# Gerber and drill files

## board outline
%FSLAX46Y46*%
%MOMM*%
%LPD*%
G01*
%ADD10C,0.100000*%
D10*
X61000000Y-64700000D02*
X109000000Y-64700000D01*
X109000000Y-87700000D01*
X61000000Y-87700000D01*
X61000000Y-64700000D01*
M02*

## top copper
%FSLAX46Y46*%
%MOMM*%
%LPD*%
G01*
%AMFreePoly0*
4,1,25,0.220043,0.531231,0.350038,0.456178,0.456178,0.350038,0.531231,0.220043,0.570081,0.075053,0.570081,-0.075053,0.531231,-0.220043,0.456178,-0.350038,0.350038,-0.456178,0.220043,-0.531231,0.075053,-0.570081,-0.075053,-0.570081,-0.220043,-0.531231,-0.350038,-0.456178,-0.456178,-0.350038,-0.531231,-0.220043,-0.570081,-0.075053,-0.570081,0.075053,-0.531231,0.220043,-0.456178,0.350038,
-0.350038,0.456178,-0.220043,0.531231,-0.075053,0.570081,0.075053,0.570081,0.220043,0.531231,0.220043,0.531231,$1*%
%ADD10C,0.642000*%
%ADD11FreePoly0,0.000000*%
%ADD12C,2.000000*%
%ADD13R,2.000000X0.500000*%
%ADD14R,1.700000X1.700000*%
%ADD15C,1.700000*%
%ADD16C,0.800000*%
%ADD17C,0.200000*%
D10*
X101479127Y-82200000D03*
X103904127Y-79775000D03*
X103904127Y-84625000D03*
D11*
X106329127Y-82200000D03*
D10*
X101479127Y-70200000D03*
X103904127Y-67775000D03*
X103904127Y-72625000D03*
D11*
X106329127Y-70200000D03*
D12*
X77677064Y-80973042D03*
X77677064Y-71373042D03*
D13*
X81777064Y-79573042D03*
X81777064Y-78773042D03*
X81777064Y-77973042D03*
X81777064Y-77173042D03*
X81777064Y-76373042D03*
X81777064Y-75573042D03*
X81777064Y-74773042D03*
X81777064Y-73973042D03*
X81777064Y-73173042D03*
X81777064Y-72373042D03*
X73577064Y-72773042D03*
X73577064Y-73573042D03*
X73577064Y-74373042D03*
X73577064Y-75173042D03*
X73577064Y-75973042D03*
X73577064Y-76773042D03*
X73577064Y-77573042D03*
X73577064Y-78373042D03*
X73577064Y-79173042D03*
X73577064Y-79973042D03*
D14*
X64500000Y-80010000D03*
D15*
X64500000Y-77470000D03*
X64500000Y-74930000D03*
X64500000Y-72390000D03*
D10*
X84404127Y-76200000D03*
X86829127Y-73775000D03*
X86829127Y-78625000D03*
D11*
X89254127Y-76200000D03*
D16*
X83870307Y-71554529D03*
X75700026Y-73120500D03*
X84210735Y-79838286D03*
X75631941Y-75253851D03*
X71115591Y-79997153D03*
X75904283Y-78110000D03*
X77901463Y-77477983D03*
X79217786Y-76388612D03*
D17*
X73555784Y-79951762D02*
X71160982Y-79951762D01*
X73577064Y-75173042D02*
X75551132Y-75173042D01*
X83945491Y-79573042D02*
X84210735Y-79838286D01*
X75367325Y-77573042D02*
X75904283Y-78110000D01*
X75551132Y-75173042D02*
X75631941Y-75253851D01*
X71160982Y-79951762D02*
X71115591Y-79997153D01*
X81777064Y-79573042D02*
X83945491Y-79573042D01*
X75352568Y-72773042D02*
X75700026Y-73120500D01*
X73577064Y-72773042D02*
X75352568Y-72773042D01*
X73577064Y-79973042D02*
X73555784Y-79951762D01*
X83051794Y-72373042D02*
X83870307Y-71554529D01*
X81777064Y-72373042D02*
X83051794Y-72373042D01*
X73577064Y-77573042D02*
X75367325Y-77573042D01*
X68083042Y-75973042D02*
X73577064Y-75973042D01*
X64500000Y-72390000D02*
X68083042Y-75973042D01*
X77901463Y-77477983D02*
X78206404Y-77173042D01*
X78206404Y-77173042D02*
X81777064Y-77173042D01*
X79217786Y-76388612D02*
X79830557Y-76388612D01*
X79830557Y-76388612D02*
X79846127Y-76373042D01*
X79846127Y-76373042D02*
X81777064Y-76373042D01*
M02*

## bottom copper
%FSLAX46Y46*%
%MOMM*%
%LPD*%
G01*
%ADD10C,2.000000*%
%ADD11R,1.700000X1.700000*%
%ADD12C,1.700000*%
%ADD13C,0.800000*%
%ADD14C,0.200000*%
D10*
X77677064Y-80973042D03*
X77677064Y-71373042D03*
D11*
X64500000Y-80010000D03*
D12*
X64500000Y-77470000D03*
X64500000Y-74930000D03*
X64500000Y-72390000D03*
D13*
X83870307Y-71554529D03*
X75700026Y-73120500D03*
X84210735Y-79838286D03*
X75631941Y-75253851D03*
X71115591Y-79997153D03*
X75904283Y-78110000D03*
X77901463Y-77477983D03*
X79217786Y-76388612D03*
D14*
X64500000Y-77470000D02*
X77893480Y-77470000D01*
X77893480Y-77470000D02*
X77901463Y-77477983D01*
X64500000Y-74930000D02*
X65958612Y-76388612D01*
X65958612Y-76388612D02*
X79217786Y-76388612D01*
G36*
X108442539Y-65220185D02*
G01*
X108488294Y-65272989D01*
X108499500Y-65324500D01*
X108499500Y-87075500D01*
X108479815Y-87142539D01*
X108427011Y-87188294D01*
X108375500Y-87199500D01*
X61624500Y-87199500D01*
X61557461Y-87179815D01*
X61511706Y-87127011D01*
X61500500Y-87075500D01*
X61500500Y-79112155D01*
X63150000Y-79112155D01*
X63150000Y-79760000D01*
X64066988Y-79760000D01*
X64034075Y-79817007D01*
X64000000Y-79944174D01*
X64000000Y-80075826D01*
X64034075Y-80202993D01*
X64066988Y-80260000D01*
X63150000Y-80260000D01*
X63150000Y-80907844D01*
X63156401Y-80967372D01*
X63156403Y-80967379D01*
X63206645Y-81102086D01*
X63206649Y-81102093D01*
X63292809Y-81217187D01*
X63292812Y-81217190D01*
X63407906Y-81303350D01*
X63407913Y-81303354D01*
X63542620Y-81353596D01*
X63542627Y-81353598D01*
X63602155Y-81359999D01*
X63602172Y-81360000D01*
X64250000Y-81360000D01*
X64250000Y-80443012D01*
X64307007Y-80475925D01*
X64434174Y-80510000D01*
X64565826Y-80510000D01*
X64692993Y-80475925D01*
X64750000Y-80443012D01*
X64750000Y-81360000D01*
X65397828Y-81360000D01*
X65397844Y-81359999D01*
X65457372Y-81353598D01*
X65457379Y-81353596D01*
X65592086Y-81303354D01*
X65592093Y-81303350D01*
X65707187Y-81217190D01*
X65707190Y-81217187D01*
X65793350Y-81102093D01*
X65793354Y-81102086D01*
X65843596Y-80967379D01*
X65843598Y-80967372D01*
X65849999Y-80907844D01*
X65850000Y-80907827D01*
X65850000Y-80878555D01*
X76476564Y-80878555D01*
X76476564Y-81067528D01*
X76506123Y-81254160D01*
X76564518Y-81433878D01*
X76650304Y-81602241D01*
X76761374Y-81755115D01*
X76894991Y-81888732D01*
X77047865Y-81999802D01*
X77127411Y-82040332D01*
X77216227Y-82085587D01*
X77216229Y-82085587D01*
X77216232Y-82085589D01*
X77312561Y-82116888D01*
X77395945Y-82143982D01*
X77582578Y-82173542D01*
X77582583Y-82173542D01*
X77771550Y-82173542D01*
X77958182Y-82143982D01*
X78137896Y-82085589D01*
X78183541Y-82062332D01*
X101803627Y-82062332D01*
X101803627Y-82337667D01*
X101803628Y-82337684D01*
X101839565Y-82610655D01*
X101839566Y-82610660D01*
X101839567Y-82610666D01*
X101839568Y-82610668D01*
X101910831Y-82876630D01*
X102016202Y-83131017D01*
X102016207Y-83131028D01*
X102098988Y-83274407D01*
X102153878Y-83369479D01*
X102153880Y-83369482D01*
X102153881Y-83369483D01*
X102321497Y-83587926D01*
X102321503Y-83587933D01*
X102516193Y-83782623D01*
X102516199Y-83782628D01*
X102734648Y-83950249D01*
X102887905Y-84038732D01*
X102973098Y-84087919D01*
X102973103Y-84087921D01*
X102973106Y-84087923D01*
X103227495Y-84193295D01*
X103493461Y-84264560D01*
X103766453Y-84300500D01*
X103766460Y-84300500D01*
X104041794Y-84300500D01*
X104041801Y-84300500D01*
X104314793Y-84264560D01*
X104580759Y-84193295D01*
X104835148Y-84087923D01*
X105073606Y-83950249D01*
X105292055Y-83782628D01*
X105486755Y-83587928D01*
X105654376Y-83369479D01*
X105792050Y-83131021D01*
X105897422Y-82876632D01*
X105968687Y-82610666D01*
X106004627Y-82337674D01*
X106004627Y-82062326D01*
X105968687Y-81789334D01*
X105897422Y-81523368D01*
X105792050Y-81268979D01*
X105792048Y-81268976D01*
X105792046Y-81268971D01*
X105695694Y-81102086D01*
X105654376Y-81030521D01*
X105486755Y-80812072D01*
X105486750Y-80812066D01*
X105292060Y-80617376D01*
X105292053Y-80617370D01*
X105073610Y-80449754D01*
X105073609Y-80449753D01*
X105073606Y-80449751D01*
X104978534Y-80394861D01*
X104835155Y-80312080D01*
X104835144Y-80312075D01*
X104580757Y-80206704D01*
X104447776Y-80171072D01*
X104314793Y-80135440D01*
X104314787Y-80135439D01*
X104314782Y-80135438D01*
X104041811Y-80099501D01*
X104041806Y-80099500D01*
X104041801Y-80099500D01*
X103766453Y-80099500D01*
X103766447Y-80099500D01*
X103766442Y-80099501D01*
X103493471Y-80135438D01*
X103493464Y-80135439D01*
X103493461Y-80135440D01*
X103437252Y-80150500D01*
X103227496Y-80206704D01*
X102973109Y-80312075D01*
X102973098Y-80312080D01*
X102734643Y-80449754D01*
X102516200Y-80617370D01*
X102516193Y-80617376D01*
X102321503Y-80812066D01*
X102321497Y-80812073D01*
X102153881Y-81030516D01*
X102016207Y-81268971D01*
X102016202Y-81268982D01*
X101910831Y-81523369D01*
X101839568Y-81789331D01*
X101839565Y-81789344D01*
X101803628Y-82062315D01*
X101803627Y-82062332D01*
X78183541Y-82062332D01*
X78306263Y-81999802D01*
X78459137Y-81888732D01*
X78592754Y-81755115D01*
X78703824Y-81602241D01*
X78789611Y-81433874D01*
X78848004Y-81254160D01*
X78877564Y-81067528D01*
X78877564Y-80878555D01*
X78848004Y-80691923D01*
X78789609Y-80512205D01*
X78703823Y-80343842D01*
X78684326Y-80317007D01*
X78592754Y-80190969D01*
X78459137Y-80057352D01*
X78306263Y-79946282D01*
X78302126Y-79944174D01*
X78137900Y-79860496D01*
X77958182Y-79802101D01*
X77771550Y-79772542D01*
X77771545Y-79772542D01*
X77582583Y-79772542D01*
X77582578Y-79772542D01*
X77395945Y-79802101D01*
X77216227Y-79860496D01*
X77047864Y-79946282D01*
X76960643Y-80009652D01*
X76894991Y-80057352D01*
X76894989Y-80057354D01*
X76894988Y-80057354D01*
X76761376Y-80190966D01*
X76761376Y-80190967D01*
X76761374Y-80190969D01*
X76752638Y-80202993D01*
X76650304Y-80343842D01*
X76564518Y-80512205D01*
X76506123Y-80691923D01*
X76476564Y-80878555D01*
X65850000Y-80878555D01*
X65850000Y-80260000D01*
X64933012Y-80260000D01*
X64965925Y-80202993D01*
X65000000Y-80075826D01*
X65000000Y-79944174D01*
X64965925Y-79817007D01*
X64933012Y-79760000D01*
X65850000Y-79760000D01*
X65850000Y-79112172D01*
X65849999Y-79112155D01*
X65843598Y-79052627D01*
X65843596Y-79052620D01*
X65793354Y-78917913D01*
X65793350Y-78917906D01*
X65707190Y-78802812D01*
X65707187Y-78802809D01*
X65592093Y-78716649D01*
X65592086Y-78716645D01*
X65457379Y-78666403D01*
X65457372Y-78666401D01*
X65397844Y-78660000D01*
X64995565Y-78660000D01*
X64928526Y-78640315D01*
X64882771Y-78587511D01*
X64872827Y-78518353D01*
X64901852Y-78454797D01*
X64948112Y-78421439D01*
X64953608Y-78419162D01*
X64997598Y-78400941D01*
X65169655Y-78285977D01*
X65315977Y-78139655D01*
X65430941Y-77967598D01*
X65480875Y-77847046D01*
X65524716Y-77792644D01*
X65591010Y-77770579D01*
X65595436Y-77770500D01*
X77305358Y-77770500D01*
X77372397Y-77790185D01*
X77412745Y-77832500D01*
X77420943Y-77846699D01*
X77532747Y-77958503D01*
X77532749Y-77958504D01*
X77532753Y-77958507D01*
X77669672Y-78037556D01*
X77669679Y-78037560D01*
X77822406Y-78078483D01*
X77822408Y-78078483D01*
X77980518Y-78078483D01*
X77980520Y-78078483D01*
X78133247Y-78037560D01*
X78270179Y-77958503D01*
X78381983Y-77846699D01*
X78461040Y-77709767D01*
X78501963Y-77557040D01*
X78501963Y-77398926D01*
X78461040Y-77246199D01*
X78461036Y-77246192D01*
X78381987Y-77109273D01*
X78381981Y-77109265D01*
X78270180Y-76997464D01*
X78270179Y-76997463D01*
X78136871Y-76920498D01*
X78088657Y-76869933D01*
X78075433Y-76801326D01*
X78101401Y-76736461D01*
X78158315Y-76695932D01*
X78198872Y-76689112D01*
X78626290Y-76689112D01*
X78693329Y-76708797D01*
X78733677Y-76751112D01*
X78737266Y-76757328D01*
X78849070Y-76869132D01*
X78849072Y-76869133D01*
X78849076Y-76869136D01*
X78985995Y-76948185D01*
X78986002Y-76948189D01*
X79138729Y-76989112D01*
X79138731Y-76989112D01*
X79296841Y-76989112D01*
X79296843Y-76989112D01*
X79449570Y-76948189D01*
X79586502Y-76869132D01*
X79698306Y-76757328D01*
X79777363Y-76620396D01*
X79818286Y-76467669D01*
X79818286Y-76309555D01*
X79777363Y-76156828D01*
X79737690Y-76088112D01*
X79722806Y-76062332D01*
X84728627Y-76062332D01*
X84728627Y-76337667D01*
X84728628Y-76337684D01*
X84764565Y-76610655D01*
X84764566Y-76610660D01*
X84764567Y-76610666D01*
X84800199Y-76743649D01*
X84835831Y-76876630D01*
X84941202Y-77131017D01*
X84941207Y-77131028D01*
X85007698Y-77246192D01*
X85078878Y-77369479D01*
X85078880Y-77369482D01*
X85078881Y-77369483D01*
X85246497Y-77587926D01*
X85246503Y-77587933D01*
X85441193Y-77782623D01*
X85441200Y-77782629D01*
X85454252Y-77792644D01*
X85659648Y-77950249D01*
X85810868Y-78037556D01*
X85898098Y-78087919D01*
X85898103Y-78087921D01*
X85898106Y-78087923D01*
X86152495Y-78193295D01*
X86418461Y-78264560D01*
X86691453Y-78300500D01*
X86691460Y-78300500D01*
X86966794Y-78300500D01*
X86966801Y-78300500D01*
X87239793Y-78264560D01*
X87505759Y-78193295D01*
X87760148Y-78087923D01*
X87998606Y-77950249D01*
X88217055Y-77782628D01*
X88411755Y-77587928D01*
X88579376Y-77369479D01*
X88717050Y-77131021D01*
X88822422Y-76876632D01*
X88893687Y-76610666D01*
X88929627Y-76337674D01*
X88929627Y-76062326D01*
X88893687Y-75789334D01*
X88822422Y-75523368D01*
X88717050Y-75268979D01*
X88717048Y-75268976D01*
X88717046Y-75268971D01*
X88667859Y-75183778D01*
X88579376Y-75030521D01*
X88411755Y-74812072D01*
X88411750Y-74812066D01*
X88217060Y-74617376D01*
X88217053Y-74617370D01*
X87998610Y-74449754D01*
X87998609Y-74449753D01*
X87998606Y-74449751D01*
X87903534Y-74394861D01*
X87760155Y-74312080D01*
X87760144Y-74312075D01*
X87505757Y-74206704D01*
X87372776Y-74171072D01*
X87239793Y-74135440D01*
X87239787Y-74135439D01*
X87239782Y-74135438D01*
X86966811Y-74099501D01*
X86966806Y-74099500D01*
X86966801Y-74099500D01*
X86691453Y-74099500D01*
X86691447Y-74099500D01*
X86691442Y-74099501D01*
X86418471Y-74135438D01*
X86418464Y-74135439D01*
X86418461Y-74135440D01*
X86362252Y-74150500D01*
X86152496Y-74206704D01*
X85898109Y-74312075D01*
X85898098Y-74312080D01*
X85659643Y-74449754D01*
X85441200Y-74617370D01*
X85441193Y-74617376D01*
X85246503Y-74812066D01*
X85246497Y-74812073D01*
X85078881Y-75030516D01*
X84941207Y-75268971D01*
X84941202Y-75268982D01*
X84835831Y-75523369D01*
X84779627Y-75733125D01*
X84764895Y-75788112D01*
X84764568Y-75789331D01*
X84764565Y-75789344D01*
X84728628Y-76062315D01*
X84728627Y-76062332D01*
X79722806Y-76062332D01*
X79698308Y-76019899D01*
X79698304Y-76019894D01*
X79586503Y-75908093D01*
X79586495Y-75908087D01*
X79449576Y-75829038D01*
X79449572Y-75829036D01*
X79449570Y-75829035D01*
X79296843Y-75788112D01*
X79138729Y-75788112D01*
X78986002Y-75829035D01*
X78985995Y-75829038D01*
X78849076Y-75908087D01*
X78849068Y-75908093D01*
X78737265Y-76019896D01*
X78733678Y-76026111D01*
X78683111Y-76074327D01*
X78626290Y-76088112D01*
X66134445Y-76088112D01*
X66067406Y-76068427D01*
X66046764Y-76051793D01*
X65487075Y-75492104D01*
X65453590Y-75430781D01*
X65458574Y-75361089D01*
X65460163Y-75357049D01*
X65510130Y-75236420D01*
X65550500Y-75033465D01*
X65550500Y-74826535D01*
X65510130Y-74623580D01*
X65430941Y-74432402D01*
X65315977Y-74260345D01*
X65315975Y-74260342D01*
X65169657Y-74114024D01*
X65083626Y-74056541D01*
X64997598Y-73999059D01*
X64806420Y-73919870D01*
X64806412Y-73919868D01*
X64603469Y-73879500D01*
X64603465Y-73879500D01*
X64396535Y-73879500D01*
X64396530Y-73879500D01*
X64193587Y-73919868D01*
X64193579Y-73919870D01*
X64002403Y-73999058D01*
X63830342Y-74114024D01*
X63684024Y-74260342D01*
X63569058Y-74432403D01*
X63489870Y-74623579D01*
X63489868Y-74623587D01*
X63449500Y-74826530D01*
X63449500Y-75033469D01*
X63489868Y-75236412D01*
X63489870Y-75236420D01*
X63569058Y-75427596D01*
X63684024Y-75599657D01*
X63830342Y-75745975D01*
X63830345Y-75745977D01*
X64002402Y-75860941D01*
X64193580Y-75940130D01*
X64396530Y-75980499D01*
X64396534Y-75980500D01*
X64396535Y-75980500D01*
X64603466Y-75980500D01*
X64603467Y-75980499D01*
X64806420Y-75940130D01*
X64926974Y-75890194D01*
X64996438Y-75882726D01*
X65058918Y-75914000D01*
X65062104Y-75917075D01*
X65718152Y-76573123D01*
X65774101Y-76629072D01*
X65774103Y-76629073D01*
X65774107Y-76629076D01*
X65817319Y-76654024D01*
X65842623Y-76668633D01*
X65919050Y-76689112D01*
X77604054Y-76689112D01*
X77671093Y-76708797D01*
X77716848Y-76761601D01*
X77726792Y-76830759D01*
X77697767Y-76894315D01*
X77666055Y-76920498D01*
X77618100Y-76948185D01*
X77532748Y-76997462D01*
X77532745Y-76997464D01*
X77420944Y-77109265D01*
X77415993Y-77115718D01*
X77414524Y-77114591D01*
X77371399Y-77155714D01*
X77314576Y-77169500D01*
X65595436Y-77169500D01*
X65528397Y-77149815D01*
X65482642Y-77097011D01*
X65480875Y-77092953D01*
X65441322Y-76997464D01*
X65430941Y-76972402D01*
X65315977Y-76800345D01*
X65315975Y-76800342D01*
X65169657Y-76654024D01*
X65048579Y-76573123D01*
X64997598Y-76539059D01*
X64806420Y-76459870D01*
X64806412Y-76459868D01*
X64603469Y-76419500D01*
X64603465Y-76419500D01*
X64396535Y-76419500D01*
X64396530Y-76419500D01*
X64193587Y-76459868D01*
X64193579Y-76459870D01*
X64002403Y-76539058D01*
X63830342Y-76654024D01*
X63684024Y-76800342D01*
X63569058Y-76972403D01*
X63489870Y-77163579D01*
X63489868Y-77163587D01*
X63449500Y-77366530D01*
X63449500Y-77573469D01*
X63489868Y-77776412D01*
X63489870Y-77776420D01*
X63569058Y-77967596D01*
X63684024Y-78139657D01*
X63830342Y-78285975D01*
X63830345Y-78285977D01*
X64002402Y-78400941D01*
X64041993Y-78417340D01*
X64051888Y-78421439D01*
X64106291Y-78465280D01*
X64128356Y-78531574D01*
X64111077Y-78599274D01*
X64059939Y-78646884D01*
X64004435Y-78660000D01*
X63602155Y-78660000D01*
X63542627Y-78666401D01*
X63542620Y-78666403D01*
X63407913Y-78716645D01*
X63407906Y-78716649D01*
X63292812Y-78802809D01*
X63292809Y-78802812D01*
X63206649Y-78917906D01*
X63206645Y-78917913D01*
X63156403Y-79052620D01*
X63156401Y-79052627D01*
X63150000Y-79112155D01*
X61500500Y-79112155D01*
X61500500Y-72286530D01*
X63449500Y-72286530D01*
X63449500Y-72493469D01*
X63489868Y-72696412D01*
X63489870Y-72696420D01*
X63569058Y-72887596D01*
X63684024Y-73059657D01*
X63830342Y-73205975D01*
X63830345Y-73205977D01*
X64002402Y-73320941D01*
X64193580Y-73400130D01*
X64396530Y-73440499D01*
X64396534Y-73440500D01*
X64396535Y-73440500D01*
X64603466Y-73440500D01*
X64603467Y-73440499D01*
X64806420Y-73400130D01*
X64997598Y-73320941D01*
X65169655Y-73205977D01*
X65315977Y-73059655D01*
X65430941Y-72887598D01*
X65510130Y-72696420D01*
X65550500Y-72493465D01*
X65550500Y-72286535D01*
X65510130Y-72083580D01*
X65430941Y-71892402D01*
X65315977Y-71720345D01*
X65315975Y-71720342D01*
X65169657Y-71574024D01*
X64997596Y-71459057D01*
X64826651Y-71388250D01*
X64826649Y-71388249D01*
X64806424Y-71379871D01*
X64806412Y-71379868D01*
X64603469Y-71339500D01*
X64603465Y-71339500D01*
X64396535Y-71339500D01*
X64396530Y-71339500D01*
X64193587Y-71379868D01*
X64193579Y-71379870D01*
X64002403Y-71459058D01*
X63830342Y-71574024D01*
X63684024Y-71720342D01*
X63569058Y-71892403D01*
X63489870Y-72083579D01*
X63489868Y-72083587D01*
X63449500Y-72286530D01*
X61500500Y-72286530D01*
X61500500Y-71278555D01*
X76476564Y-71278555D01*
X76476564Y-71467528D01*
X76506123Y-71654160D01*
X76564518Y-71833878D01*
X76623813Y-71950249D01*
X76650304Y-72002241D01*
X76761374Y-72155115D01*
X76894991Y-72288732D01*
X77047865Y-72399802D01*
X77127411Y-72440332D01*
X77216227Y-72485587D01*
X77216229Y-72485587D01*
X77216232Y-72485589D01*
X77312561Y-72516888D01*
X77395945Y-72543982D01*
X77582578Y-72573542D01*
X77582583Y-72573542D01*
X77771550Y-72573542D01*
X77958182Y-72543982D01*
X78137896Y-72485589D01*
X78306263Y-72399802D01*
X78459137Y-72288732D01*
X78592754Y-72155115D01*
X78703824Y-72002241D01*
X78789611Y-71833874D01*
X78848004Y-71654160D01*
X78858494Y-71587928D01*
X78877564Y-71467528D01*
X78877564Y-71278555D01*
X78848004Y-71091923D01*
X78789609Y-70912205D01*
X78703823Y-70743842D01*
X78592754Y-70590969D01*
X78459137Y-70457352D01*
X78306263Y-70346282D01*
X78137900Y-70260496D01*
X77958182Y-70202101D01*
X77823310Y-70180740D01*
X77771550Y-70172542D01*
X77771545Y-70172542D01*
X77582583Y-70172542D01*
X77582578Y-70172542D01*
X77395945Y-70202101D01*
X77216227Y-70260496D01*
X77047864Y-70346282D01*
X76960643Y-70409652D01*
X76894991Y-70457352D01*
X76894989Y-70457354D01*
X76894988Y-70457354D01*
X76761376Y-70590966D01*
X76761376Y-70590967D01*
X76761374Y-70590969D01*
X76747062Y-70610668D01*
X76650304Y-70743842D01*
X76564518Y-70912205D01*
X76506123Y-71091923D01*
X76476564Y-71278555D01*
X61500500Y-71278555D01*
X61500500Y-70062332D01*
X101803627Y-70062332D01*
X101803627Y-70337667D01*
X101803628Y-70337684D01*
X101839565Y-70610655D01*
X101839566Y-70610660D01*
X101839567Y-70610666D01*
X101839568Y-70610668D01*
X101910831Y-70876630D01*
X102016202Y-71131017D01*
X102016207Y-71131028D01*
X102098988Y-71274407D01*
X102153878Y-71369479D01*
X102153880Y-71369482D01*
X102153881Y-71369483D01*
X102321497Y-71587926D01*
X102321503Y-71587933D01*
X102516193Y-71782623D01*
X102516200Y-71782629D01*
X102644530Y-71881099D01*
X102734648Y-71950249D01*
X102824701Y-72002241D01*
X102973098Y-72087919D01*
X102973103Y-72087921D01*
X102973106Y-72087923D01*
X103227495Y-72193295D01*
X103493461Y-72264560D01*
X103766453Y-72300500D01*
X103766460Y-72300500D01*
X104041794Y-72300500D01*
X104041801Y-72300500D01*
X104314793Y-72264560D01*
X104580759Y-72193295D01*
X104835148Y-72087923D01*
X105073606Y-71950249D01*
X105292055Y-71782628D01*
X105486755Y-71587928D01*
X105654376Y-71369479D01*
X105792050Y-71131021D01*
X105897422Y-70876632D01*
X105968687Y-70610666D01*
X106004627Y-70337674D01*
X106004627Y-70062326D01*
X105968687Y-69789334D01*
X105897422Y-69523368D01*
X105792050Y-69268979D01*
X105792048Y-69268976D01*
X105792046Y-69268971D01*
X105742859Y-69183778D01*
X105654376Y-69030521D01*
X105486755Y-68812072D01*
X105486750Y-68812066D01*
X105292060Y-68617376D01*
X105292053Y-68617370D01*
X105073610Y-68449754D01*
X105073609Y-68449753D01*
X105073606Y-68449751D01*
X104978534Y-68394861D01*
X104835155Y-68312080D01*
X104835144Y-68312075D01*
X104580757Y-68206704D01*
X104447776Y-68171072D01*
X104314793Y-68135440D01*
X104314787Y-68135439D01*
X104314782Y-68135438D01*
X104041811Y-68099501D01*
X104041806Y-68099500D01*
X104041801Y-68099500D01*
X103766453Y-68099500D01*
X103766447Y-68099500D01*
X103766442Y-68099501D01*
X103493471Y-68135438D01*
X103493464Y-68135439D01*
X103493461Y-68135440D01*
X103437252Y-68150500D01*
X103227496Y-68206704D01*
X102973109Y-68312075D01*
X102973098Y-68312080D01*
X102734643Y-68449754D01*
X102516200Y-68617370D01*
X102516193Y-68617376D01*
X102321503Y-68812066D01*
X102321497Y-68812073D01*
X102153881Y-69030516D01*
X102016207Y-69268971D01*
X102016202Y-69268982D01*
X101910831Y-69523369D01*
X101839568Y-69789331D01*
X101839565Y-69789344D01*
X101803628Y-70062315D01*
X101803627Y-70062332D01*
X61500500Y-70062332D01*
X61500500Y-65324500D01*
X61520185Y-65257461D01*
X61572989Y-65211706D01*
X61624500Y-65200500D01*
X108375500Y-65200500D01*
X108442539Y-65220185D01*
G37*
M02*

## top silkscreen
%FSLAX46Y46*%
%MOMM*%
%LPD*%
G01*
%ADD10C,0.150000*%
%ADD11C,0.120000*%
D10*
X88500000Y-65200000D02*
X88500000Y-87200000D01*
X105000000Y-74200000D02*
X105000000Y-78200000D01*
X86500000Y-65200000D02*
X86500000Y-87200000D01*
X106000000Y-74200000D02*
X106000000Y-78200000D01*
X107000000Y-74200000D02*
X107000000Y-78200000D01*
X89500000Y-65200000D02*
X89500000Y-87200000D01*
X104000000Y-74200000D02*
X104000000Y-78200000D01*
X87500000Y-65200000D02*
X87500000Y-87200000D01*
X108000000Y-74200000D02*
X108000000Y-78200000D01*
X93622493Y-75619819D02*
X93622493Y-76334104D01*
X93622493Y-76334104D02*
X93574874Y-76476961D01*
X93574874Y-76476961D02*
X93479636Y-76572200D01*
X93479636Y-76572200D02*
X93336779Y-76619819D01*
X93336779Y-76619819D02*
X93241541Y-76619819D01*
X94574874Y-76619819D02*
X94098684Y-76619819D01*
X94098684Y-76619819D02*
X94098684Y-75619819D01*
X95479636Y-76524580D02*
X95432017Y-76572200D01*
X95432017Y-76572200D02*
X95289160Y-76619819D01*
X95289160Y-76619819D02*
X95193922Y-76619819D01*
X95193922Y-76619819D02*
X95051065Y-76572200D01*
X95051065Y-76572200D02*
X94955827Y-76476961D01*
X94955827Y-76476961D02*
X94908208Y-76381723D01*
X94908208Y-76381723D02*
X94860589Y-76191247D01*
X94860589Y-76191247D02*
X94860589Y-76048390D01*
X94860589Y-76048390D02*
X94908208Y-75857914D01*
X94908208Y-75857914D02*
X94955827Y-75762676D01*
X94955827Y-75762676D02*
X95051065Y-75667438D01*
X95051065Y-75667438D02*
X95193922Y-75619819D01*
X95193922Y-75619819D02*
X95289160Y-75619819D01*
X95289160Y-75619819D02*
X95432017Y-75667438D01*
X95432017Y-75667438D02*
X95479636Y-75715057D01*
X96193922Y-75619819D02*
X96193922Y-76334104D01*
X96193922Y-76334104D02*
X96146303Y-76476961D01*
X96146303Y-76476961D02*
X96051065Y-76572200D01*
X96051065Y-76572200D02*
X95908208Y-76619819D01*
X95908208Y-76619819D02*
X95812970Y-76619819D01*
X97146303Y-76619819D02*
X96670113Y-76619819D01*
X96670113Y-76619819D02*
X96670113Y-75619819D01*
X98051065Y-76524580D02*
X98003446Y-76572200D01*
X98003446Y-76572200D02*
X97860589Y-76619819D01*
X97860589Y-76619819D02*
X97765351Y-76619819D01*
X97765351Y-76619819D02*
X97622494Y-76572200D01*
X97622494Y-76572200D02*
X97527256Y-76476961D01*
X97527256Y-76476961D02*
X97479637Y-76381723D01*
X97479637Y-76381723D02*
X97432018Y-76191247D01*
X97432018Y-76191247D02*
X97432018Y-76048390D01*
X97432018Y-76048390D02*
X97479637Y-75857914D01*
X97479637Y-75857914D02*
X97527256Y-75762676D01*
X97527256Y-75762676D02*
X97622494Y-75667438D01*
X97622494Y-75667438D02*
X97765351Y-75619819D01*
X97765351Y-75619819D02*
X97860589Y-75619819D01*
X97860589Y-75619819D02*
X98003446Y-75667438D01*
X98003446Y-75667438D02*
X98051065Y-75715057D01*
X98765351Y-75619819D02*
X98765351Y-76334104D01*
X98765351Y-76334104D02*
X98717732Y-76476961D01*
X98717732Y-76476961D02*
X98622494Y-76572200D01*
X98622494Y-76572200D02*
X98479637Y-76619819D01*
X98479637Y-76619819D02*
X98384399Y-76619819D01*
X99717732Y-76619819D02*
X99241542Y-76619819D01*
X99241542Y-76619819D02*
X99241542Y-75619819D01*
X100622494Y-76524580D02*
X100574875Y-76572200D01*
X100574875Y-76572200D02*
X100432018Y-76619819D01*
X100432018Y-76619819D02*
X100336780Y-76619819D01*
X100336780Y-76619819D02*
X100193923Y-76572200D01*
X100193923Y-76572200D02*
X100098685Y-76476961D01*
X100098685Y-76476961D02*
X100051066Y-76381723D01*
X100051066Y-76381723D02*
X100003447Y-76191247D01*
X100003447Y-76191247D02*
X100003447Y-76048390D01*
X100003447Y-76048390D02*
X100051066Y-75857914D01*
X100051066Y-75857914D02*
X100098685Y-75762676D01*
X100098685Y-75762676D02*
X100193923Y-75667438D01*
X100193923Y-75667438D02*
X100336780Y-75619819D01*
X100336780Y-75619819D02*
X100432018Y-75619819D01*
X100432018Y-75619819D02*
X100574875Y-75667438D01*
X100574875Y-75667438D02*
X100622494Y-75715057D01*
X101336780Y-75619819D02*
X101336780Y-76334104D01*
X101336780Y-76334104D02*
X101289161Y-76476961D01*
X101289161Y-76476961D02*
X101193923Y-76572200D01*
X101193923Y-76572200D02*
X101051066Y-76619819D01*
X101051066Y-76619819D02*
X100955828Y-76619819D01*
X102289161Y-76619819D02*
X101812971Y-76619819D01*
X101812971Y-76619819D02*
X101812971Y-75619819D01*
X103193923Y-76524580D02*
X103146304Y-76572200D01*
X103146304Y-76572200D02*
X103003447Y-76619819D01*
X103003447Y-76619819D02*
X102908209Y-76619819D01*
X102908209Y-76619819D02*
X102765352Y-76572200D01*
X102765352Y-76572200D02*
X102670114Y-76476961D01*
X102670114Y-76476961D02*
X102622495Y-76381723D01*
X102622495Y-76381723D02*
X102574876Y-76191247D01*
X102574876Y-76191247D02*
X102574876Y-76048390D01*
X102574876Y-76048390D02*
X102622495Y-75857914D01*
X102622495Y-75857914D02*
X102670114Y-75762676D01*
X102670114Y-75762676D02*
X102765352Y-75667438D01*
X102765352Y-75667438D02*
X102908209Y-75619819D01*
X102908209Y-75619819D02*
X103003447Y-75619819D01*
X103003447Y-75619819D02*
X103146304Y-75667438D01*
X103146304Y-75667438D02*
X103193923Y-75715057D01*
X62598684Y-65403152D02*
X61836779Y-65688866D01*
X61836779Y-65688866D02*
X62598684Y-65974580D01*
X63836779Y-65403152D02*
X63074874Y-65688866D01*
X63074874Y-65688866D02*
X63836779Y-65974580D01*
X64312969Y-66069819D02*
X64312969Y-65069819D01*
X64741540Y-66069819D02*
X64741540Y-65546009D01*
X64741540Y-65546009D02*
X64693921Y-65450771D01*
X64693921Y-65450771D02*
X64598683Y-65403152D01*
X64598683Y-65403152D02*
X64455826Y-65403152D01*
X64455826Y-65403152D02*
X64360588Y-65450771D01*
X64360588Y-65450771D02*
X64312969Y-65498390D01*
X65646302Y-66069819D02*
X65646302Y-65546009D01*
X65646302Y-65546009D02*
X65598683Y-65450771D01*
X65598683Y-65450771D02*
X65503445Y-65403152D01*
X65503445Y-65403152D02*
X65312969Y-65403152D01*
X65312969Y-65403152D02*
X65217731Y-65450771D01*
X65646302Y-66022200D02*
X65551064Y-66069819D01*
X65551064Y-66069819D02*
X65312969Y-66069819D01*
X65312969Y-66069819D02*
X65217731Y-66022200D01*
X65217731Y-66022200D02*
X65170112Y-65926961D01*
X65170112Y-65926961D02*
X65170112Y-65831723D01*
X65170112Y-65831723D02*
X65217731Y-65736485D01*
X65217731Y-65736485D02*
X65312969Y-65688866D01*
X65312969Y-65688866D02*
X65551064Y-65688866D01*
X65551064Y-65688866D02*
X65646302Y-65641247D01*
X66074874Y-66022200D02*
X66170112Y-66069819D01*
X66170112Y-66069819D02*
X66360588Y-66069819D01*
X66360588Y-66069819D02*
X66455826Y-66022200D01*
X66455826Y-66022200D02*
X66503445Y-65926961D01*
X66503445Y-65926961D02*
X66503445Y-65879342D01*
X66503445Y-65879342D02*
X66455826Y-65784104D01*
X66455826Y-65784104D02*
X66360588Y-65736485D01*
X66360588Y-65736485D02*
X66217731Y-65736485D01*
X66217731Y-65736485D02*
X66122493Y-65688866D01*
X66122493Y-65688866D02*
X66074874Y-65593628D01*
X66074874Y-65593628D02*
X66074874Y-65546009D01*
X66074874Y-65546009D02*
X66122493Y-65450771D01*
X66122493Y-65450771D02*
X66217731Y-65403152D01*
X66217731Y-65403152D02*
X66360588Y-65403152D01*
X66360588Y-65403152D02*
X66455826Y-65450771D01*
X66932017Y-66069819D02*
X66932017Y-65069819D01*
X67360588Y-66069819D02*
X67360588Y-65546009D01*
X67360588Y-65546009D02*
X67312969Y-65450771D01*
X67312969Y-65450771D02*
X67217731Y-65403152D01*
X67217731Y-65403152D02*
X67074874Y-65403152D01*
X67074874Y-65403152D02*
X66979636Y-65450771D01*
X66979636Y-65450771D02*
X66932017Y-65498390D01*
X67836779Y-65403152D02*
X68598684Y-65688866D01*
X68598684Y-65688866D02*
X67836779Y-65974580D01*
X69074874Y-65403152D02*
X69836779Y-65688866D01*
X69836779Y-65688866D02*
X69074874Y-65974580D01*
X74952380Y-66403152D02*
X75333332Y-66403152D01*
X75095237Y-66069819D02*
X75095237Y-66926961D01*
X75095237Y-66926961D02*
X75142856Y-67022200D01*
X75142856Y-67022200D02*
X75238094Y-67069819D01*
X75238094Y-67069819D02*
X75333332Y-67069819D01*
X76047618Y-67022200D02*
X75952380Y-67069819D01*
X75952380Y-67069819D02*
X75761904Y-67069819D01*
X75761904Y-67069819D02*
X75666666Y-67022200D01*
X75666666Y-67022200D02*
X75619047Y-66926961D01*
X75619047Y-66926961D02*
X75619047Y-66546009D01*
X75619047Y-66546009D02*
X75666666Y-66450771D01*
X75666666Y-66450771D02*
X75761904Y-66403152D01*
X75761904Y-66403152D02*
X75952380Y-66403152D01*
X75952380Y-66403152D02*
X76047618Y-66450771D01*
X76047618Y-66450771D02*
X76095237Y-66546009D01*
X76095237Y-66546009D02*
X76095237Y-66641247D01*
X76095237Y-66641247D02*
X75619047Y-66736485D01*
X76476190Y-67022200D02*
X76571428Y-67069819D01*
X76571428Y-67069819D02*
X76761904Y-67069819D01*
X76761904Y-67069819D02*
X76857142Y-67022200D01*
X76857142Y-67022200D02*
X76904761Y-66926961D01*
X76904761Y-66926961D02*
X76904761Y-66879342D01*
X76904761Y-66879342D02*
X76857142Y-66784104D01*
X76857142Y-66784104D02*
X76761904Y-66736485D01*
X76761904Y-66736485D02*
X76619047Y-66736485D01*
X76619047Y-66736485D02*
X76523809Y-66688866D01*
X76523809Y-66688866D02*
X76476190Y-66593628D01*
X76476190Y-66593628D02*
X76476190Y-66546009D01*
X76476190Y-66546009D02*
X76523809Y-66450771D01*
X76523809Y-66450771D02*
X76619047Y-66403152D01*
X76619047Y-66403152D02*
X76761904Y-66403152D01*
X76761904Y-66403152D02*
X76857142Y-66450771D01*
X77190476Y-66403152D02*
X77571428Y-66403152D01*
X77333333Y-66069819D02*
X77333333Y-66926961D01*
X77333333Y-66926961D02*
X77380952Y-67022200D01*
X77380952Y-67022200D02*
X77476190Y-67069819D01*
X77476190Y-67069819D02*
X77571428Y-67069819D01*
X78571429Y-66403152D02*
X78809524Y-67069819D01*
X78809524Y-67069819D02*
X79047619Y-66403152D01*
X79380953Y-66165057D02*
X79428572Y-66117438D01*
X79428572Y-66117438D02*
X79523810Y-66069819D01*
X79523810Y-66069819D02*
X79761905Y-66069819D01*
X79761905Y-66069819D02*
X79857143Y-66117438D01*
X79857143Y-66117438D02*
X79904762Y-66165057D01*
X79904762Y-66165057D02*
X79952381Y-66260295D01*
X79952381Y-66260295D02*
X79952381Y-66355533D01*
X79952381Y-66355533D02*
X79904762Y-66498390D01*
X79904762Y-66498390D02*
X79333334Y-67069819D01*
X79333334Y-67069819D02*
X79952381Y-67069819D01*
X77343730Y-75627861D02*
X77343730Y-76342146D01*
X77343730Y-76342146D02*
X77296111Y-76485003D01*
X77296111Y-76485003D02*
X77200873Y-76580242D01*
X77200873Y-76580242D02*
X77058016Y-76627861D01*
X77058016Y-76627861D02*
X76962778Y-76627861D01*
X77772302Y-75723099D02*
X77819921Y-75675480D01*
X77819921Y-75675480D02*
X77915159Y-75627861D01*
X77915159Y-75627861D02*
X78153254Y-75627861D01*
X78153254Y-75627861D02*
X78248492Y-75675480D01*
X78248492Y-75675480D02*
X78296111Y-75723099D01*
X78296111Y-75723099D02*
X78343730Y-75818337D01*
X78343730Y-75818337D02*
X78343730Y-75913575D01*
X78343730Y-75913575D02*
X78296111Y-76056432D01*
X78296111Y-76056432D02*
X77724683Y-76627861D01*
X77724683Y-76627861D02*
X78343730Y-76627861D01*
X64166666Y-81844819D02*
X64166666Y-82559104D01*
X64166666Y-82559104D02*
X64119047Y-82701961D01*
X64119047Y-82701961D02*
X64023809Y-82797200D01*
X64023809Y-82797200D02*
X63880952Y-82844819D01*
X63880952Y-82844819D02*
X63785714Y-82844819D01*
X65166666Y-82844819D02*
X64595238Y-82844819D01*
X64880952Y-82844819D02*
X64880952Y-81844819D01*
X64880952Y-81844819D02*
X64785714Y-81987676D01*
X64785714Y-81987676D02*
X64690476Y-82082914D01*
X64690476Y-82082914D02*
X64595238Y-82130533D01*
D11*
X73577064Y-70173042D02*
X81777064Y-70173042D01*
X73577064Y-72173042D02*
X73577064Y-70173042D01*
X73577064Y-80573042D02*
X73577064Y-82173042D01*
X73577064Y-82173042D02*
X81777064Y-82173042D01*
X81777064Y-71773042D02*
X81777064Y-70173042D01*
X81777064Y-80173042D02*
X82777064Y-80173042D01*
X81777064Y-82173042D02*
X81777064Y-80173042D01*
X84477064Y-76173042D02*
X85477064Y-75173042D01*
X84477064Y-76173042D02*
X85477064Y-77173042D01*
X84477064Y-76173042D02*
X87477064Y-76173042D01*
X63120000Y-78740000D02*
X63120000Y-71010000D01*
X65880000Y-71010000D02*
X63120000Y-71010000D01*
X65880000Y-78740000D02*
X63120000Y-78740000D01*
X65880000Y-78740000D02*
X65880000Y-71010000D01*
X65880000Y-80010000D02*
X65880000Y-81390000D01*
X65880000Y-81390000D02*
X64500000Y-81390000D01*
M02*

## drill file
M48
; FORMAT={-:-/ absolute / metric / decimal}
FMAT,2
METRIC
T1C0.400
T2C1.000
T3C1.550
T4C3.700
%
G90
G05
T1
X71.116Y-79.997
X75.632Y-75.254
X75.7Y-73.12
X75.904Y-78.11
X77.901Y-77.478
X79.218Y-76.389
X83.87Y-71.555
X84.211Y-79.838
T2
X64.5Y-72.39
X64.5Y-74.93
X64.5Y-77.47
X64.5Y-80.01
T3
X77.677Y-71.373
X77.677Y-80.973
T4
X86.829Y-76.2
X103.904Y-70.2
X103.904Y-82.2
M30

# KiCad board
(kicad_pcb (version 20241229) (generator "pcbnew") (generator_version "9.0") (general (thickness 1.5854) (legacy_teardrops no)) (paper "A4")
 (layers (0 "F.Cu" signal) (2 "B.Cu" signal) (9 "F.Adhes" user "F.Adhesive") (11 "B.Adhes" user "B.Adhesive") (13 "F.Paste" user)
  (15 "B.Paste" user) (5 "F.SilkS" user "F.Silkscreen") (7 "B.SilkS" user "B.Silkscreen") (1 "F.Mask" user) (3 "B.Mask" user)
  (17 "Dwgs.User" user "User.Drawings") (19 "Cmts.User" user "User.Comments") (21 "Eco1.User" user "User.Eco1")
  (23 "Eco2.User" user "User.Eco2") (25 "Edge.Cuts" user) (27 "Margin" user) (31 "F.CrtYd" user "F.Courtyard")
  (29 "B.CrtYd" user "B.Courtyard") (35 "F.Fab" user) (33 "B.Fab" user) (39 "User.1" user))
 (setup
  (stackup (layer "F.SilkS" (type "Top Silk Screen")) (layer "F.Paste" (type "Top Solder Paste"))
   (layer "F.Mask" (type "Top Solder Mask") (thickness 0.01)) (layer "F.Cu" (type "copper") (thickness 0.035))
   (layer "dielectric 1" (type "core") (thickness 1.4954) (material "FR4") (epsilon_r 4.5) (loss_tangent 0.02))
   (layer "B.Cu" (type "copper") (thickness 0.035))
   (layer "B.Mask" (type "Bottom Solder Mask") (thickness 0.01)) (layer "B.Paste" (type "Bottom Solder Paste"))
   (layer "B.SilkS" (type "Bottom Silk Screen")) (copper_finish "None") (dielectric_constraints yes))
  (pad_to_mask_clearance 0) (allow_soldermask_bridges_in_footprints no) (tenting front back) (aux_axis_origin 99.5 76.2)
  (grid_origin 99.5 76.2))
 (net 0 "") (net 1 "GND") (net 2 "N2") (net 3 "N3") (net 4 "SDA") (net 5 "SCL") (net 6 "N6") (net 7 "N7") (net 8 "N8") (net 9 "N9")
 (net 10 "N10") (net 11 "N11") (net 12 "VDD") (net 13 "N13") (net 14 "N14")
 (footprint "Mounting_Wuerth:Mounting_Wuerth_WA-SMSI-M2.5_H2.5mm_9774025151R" (layer "F.Cu") (at 103.904127 82.2)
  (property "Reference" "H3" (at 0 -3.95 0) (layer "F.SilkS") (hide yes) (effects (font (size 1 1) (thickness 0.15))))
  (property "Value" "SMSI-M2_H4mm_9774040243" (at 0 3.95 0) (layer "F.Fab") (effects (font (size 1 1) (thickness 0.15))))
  (pad "" smd custom (at -1.704127 -1.704127) (size 0.51 0.51) (layers "F.Paste") (options (clearance outline) (anchor circle)) (primitives))
  (pad "" smd custom (at -1.704127 1.704127) (size 0.51 0.51) (layers "F.Paste") (options (clearance outline) (anchor circle)) (primitives))
  (pad "" np_thru_hole circle (at 0 0) (size 3.7 3.7) (drill 3.7) (layers "*.Cu" "*.Mask"))
  (pad "" smd custom (at 1.704127 -1.704127) (size 0.51 0.51) (layers "F.Paste") (options (clearance outline) (anchor circle)) (primitives))
  (pad "" smd custom (at 1.704127 1.704127) (size 0.51 0.51) (layers "F.Paste") (options (clearance outline) (anchor circle)) (primitives))
  (pad "1" smd circle (at -2.425 0) (size 0.642 0.642) (layers "F.Cu"))
  (pad "1" smd circle (at 0 -2.425) (size 0.642 0.642) (layers "F.Cu"))
  (pad "1" smd circle (at 0 2.425) (size 0.642 0.642) (layers "F.Cu"))
  (pad "1" smd custom (at 2.425 0) (size 1.15 1.15) (layers "F.Cu" "F.Mask") (options (clearance outline) (anchor circle)) (primitives)))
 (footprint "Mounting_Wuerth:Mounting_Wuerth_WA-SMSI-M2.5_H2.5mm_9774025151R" (layer "F.Cu") (at 103.904127 70.2)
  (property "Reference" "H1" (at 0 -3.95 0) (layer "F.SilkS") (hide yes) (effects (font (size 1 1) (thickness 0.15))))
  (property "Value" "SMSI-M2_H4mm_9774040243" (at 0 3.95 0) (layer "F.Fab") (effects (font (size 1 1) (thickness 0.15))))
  (pad "" smd custom (at -1.704127 -1.704127) (size 0.51 0.51) (layers "F.Paste") (options (clearance outline) (anchor circle)) (primitives))
  (pad "" smd custom (at -1.704127 1.704127) (size 0.51 0.51) (layers "F.Paste") (options (clearance outline) (anchor circle)) (primitives))
  (pad "" np_thru_hole circle (at 0 0) (size 3.7 3.7) (drill 3.7) (layers "*.Cu" "*.Mask"))
  (pad "" smd custom (at 1.704127 -1.704127) (size 0.51 0.51) (layers "F.Paste") (options (clearance outline) (anchor circle)) (primitives))
  (pad "" smd custom (at 1.704127 1.704127) (size 0.51 0.51) (layers "F.Paste") (options (clearance outline) (anchor circle)) (primitives))
  (pad "1" smd circle (at -2.425 0) (size 0.642 0.642) (layers "F.Cu"))
  (pad "1" smd circle (at 0 -2.425) (size 0.642 0.642) (layers "F.Cu"))
  (pad "1" smd circle (at 0 2.425) (size 0.642 0.642) (layers "F.Cu"))
  (pad "1" smd custom (at 2.425 0) (size 1.15 1.15) (layers "F.Cu" "F.Mask") (options (clearance outline) (anchor circle)) (primitives)))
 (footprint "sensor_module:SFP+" (layer "F.Cu") (at 71.477064 76.173042 180)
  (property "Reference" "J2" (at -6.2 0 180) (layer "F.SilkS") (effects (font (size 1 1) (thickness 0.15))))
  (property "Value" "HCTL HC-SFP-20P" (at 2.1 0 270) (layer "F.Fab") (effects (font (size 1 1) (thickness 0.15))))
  (fp_line (start -2.1 6) (end -10.3 6) (stroke (width 0.12) (type solid)) (layer "F.SilkS"))
  (fp_line (start -2.1 4) (end -2.1 6) (stroke (width 0.12) (type solid)) (layer "F.SilkS"))
  (fp_line (start -2.1 -4.4) (end -2.1 -6) (stroke (width 0.12) (type solid)) (layer "F.SilkS"))
  (fp_line (start -2.1 -6) (end -10.3 -6) (stroke (width 0.12) (type solid)) (layer "F.SilkS"))
  (fp_line (start -10.3 4.4) (end -10.3 6) (stroke (width 0.12) (type solid)) (layer "F.SilkS"))
  (fp_line (start -10.3 -4) (end -11.3 -4) (stroke (width 0.12) (type solid)) (layer "F.SilkS"))
  (fp_line (start -10.3 -6) (end -10.3 -4) (stroke (width 0.12) (type solid)) (layer "F.SilkS"))
  (fp_line (start -13 0) (end -14 1) (stroke (width 0.12) (type solid)) (layer "F.SilkS"))
  (fp_line (start -13 0) (end -14 -1) (stroke (width 0.12) (type solid)) (layer "F.SilkS"))
  (fp_line (start -13 0) (end -16 0) (stroke (width 0.12) (type solid)) (layer "F.SilkS"))
  (pad "" np_thru_hole circle (at -6.2 -4.8 180) (size 2 2) (drill 1.55) (layers "*.Cu" "*.Mask"))
  (pad "" np_thru_hole circle (at -6.2 4.8 180) (size 2 2) (drill 1.55) (layers "*.Cu" "*.Mask"))
  (pad "1" smd rect (at -10.3 -3.4 180) (size 2 0.5) (layers "F.Cu" "F.Mask" "F.Paste") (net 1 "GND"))
  (pad "2" smd rect (at -10.3 -2.6 180) (size 2 0.5) (layers "F.Cu" "F.Mask" "F.Paste") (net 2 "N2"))
  (pad "3" smd rect (at -10.3 -1.8 180) (size 2 0.5) (layers "F.Cu" "F.Mask" "F.Paste") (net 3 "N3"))
  (pad "4" smd rect (at -10.3 -1 180) (size 2 0.5) (layers "F.Cu" "F.Mask" "F.Paste") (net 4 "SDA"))
  (pad "5" smd rect (at -10.3 -0.2 180) (size 2 0.5) (layers "F.Cu" "F.Mask" "F.Paste") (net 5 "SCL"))
  (pad "6" smd rect (at -10.3 0.6 180) (size 2 0.5) (layers "F.Cu" "F.Mask" "F.Paste") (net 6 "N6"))
  (pad "7" smd rect (at -10.3 1.4 180) (size 2 0.5) (layers "F.Cu" "F.Mask" "F.Paste") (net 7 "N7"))
  (pad "8" smd rect (at -10.3 2.2 180) (size 2 0.5) (layers "F.Cu" "F.Mask" "F.Paste") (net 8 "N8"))
  (pad "9" smd rect (at -10.3 3 180) (size 2 0.5) (layers "F.Cu" "F.Mask" "F.Paste") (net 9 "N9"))
  (pad "10" smd rect (at -10.3 3.8 180) (size 2 0.5) (layers "F.Cu" "F.Mask" "F.Paste") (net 1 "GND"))
  (pad "11" smd rect (at -2.1 3.4 180) (size 2 0.5) (layers "F.Cu" "F.Mask" "F.Paste") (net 1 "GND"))
  (pad "12" smd rect (at -2.1 2.6 180) (size 2 0.5) (layers "F.Cu" "F.Mask" "F.Paste") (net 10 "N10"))
  (pad "13" smd rect (at -2.1 1.8 180) (size 2 0.5) (layers "F.Cu" "F.Mask" "F.Paste") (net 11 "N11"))
  (pad "14" smd rect (at -2.1 1 180) (size 2 0.5) (layers "F.Cu" "F.Mask" "F.Paste") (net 1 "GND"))
  (pad "15" smd rect (at -2.1 0.2 180) (size 2 0.5) (layers "F.Cu" "F.Mask" "F.Paste") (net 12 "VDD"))
  (pad "16" smd rect (at -2.1 -0.6 180) (size 2 0.5) (layers "F.Cu" "F.Mask" "F.Paste") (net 12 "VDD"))
  (pad "17" smd rect (at -2.1 -1.4 180) (size 2 0.5) (layers "F.Cu" "F.Mask" "F.Paste") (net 1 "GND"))
  (pad "18" smd rect (at -2.1 -2.2 180) (size 2 0.5) (layers "F.Cu" "F.Mask" "F.Paste") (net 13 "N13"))
  (pad "19" smd rect (at -2.1 -3 180) (size 2 0.5) (layers "F.Cu" "F.Mask" "F.Paste") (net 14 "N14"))
  (pad "20" smd rect (at -2.1 -3.8 180) (size 2 0.5) (layers "F.Cu" "F.Mask" "F.Paste") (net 1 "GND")))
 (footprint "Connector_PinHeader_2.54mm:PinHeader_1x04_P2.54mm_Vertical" (layer "F.Cu") (at 64.5 80.01 180)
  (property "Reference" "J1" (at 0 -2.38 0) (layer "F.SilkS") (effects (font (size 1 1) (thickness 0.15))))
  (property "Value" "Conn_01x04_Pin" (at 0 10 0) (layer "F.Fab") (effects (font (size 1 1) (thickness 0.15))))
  (fp_line (start 1.38 1.27) (end 1.38 9) (stroke (width 0.12) (type solid)) (layer "F.SilkS"))
  (fp_line (start -1.38 9) (end 1.38 9) (stroke (width 0.12) (type solid)) (layer "F.SilkS"))
  (fp_line (start -1.38 1.27) (end 1.38 1.27) (stroke (width 0.12) (type solid)) (layer "F.SilkS"))
  (fp_line (start -1.38 1.27) (end -1.38 9) (stroke (width 0.12) (type solid)) (layer "F.SilkS"))
  (fp_line (start -1.38 0) (end -1.38 -1.38) (stroke (width 0.12) (type solid)) (layer "F.SilkS"))
  (fp_line (start -1.38 -1.38) (end 0 -1.38) (stroke (width 0.12) (type solid)) (layer "F.SilkS"))
  (pad "1" thru_hole rect (at 0 0 180) (size 1.7 1.7) (drill 1) (layers "*.Cu" "*.Mask") (remove_unused_layers no) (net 1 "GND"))
  (pad "2" thru_hole circle (at 0 2.54 180) (size 1.7 1.7) (drill 1) (layers "*.Cu" "*.Mask") (remove_unused_layers no) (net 4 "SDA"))
  (pad "3" thru_hole circle (at 0 5.08 180) (size 1.7 1.7) (drill 1) (layers "*.Cu" "*.Mask") (remove_unused_layers no) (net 5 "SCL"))
  (pad "4" thru_hole circle (at 0 7.62 180) (size 1.7 1.7) (drill 1) (layers "*.Cu" "*.Mask") (remove_unused_layers no) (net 12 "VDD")))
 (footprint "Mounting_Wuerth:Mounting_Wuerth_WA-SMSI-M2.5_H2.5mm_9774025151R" (layer "F.Cu") (at 86.829127 76.2)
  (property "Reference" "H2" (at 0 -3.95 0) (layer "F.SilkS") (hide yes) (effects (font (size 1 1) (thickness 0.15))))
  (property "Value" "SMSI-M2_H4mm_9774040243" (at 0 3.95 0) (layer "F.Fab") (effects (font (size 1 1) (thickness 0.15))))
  (pad "" smd custom (at -1.704127 -1.704127) (size 0.51 0.51) (layers "F.Paste") (options (clearance outline) (anchor circle)) (primitives))
  (pad "" smd custom (at -1.704127 1.704127) (size 0.51 0.51) (layers "F.Paste") (options (clearance outline) (anchor circle)) (primitives))
  (pad "" np_thru_hole circle (at 0 0) (size 3.7 3.7) (drill 3.7) (layers "*.Cu" "*.Mask"))
  (pad "" smd custom (at 1.704127 -1.704127) (size 0.51 0.51) (layers "F.Paste") (options (clearance outline) (anchor circle)) (primitives))
  (pad "" smd custom (at 1.704127 1.704127) (size 0.51 0.51) (layers "F.Paste") (options (clearance outline) (anchor circle)) (primitives))
  (pad "1" smd circle (at -2.425 0) (size 0.642 0.642) (layers "F.Cu"))
  (pad "1" smd circle (at 0 -2.425) (size 0.642 0.642) (layers "F.Cu"))
  (pad "1" smd circle (at 0 2.425) (size 0.642 0.642) (layers "F.Cu"))
  (pad "1" smd custom (at 2.425 0) (size 1.15 1.15) (layers "F.Cu" "F.Mask") (options (clearance outline) (anchor circle)) (primitives)))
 (gr_line (start 88.5 65.2) (end 88.5 87.2) (stroke (width 0.15) (type default)) (layer "F.SilkS"))
 (gr_line (start 105 74.2) (end 105 78.2) (stroke (width 0.15) (type default)) (layer "F.SilkS"))
 (gr_line (start 86.5 65.2) (end 86.5 87.2) (stroke (width 0.15) (type default)) (layer "F.SilkS"))
 (gr_line (start 106 74.2) (end 106 78.2) (stroke (width 0.15) (type default)) (layer "F.SilkS"))
 (gr_line (start 107 74.2) (end 107 78.2) (stroke (width 0.15) (type default)) (layer "F.SilkS"))
 (gr_line (start 89.5 65.2) (end 89.5 87.2) (stroke (width 0.15) (type default)) (layer "F.SilkS"))
 (gr_line (start 104 74.2) (end 104 78.2) (stroke (width 0.15) (type default)) (layer "F.SilkS"))
 (gr_line (start 87.5 65.2) (end 87.5 87.2) (stroke (width 0.15) (type default)) (layer "F.SilkS"))
 (gr_line (start 108 74.2) (end 108 78.2) (stroke (width 0.15) (type default)) (layer "F.SilkS"))
 (gr_rect (start 61 64.7) (end 109 87.7) (stroke (width 0.1) (type default)) (fill no) (layer "Edge.Cuts"))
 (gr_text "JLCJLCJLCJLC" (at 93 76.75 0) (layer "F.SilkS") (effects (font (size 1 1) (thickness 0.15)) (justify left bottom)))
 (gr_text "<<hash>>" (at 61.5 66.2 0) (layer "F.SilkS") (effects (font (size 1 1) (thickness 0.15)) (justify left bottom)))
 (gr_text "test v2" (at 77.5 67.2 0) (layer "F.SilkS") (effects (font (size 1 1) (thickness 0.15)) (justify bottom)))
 (segment (start 73.555784 79.951762) (end 71.160982 79.951762) (width 0.2) (layer "F.Cu") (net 1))
 (segment (start 73.577064 75.173042) (end 75.551132 75.173042) (width 0.2) (layer "F.Cu") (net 1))
 (segment (start 83.945491 79.573042) (end 84.210735 79.838286) (width 0.2) (layer "F.Cu") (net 1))
 (segment (start 75.367325 77.573042) (end 75.904283 78.11) (width 0.2) (layer "F.Cu") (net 1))
 (segment (start 75.551132 75.173042) (end 75.631941 75.253851) (width 0.2) (layer "F.Cu") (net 1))
 (segment (start 71.160982 79.951762) (end 71.115591 79.997153) (width 0.2) (layer "F.Cu") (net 1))
 (segment (start 81.777064 79.573042) (end 83.945491 79.573042) (width 0.2) (layer "F.Cu") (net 1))
 (segment (start 75.352568 72.773042) (end 75.700026 73.1205) (width 0.2) (layer "F.Cu") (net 1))
 (segment (start 73.577064 72.773042) (end 75.352568 72.773042) (width 0.2) (layer "F.Cu") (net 1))
 (segment (start 73.577064 79.973042) (end 73.555784 79.951762) (width 0.2) (layer "F.Cu") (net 1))
 (segment (start 83.051794 72.373042) (end 83.870307 71.554529) (width 0.2) (layer "F.Cu") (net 1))
 (segment (start 81.777064 72.373042) (end 83.051794 72.373042) (width 0.2) (layer "F.Cu") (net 1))
 (segment (start 73.577064 77.573042) (end 75.367325 77.573042) (width 0.2) (layer "F.Cu") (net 1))
 (via (at 83.870307 71.554529) (size 0.8) (drill 0.4) (layers "F.Cu" "B.Cu") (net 1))
 (via (at 75.700026 73.1205) (size 0.8) (drill 0.4) (layers "F.Cu" "B.Cu") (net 1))
 (via (at 84.210735 79.838286) (size 0.8) (drill 0.4) (layers "F.Cu" "B.Cu") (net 1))
 (via (at 75.631941 75.253851) (size 0.8) (drill 0.4) (layers "F.Cu" "B.Cu") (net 1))
 (via (at 71.115591 79.997153) (size 0.8) (drill 0.4) (layers "F.Cu" "B.Cu") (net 1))
 (via (at 75.904283 78.11) (size 0.8) (drill 0.4) (layers "F.Cu" "B.Cu") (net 1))
 (segment (start 68.083042 75.973042) (end 73.577064 75.973042) (width 0.2) (layer "F.Cu") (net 12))
 (segment (start 64.5 72.39) (end 68.083042 75.973042) (width 0.2) (layer "F.Cu") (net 12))
 (segment (start 77.901463 77.477983) (end 78.206404 77.173042) (width 0.2) (layer "F.Cu") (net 4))
 (segment (start 78.206404 77.173042) (end 81.777064 77.173042) (width 0.2) (layer "F.Cu") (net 4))
 (via (at 77.901463 77.477983) (size 0.8) (drill 0.4) (layers "F.Cu" "B.Cu") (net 4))
 (segment (start 64.5 77.47) (end 77.89348 77.47) (width 0.2) (layer "B.Cu") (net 4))
 (segment (start 77.89348 77.47) (end 77.901463 77.477983) (width 0.2) (layer "B.Cu") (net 4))
 (segment (start 79.217786 76.388612) (end 79.830557 76.388612) (width 0.2) (layer "F.Cu") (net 5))
 (segment (start 79.830557 76.388612) (end 79.846127 76.373042) (width 0.2) (layer "F.Cu") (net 5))
 (segment (start 79.846127 76.373042) (end 81.777064 76.373042) (width 0.2) (layer "F.Cu") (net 5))
 (via (at 79.217786 76.388612) (size 0.8) (drill 0.4) (layers "F.Cu" "B.Cu") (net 5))
 (segment (start 64.5 74.93) (end 65.958612 76.388612) (width 0.2) (layer "B.Cu") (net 5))
 (segment (start 65.958612 76.388612) (end 79.217786 76.388612) (width 0.2) (layer "B.Cu") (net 5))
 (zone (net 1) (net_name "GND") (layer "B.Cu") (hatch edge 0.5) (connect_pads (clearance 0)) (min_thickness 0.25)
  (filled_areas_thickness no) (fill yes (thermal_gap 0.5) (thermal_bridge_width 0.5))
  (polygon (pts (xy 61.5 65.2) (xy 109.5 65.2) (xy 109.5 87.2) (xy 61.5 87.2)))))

